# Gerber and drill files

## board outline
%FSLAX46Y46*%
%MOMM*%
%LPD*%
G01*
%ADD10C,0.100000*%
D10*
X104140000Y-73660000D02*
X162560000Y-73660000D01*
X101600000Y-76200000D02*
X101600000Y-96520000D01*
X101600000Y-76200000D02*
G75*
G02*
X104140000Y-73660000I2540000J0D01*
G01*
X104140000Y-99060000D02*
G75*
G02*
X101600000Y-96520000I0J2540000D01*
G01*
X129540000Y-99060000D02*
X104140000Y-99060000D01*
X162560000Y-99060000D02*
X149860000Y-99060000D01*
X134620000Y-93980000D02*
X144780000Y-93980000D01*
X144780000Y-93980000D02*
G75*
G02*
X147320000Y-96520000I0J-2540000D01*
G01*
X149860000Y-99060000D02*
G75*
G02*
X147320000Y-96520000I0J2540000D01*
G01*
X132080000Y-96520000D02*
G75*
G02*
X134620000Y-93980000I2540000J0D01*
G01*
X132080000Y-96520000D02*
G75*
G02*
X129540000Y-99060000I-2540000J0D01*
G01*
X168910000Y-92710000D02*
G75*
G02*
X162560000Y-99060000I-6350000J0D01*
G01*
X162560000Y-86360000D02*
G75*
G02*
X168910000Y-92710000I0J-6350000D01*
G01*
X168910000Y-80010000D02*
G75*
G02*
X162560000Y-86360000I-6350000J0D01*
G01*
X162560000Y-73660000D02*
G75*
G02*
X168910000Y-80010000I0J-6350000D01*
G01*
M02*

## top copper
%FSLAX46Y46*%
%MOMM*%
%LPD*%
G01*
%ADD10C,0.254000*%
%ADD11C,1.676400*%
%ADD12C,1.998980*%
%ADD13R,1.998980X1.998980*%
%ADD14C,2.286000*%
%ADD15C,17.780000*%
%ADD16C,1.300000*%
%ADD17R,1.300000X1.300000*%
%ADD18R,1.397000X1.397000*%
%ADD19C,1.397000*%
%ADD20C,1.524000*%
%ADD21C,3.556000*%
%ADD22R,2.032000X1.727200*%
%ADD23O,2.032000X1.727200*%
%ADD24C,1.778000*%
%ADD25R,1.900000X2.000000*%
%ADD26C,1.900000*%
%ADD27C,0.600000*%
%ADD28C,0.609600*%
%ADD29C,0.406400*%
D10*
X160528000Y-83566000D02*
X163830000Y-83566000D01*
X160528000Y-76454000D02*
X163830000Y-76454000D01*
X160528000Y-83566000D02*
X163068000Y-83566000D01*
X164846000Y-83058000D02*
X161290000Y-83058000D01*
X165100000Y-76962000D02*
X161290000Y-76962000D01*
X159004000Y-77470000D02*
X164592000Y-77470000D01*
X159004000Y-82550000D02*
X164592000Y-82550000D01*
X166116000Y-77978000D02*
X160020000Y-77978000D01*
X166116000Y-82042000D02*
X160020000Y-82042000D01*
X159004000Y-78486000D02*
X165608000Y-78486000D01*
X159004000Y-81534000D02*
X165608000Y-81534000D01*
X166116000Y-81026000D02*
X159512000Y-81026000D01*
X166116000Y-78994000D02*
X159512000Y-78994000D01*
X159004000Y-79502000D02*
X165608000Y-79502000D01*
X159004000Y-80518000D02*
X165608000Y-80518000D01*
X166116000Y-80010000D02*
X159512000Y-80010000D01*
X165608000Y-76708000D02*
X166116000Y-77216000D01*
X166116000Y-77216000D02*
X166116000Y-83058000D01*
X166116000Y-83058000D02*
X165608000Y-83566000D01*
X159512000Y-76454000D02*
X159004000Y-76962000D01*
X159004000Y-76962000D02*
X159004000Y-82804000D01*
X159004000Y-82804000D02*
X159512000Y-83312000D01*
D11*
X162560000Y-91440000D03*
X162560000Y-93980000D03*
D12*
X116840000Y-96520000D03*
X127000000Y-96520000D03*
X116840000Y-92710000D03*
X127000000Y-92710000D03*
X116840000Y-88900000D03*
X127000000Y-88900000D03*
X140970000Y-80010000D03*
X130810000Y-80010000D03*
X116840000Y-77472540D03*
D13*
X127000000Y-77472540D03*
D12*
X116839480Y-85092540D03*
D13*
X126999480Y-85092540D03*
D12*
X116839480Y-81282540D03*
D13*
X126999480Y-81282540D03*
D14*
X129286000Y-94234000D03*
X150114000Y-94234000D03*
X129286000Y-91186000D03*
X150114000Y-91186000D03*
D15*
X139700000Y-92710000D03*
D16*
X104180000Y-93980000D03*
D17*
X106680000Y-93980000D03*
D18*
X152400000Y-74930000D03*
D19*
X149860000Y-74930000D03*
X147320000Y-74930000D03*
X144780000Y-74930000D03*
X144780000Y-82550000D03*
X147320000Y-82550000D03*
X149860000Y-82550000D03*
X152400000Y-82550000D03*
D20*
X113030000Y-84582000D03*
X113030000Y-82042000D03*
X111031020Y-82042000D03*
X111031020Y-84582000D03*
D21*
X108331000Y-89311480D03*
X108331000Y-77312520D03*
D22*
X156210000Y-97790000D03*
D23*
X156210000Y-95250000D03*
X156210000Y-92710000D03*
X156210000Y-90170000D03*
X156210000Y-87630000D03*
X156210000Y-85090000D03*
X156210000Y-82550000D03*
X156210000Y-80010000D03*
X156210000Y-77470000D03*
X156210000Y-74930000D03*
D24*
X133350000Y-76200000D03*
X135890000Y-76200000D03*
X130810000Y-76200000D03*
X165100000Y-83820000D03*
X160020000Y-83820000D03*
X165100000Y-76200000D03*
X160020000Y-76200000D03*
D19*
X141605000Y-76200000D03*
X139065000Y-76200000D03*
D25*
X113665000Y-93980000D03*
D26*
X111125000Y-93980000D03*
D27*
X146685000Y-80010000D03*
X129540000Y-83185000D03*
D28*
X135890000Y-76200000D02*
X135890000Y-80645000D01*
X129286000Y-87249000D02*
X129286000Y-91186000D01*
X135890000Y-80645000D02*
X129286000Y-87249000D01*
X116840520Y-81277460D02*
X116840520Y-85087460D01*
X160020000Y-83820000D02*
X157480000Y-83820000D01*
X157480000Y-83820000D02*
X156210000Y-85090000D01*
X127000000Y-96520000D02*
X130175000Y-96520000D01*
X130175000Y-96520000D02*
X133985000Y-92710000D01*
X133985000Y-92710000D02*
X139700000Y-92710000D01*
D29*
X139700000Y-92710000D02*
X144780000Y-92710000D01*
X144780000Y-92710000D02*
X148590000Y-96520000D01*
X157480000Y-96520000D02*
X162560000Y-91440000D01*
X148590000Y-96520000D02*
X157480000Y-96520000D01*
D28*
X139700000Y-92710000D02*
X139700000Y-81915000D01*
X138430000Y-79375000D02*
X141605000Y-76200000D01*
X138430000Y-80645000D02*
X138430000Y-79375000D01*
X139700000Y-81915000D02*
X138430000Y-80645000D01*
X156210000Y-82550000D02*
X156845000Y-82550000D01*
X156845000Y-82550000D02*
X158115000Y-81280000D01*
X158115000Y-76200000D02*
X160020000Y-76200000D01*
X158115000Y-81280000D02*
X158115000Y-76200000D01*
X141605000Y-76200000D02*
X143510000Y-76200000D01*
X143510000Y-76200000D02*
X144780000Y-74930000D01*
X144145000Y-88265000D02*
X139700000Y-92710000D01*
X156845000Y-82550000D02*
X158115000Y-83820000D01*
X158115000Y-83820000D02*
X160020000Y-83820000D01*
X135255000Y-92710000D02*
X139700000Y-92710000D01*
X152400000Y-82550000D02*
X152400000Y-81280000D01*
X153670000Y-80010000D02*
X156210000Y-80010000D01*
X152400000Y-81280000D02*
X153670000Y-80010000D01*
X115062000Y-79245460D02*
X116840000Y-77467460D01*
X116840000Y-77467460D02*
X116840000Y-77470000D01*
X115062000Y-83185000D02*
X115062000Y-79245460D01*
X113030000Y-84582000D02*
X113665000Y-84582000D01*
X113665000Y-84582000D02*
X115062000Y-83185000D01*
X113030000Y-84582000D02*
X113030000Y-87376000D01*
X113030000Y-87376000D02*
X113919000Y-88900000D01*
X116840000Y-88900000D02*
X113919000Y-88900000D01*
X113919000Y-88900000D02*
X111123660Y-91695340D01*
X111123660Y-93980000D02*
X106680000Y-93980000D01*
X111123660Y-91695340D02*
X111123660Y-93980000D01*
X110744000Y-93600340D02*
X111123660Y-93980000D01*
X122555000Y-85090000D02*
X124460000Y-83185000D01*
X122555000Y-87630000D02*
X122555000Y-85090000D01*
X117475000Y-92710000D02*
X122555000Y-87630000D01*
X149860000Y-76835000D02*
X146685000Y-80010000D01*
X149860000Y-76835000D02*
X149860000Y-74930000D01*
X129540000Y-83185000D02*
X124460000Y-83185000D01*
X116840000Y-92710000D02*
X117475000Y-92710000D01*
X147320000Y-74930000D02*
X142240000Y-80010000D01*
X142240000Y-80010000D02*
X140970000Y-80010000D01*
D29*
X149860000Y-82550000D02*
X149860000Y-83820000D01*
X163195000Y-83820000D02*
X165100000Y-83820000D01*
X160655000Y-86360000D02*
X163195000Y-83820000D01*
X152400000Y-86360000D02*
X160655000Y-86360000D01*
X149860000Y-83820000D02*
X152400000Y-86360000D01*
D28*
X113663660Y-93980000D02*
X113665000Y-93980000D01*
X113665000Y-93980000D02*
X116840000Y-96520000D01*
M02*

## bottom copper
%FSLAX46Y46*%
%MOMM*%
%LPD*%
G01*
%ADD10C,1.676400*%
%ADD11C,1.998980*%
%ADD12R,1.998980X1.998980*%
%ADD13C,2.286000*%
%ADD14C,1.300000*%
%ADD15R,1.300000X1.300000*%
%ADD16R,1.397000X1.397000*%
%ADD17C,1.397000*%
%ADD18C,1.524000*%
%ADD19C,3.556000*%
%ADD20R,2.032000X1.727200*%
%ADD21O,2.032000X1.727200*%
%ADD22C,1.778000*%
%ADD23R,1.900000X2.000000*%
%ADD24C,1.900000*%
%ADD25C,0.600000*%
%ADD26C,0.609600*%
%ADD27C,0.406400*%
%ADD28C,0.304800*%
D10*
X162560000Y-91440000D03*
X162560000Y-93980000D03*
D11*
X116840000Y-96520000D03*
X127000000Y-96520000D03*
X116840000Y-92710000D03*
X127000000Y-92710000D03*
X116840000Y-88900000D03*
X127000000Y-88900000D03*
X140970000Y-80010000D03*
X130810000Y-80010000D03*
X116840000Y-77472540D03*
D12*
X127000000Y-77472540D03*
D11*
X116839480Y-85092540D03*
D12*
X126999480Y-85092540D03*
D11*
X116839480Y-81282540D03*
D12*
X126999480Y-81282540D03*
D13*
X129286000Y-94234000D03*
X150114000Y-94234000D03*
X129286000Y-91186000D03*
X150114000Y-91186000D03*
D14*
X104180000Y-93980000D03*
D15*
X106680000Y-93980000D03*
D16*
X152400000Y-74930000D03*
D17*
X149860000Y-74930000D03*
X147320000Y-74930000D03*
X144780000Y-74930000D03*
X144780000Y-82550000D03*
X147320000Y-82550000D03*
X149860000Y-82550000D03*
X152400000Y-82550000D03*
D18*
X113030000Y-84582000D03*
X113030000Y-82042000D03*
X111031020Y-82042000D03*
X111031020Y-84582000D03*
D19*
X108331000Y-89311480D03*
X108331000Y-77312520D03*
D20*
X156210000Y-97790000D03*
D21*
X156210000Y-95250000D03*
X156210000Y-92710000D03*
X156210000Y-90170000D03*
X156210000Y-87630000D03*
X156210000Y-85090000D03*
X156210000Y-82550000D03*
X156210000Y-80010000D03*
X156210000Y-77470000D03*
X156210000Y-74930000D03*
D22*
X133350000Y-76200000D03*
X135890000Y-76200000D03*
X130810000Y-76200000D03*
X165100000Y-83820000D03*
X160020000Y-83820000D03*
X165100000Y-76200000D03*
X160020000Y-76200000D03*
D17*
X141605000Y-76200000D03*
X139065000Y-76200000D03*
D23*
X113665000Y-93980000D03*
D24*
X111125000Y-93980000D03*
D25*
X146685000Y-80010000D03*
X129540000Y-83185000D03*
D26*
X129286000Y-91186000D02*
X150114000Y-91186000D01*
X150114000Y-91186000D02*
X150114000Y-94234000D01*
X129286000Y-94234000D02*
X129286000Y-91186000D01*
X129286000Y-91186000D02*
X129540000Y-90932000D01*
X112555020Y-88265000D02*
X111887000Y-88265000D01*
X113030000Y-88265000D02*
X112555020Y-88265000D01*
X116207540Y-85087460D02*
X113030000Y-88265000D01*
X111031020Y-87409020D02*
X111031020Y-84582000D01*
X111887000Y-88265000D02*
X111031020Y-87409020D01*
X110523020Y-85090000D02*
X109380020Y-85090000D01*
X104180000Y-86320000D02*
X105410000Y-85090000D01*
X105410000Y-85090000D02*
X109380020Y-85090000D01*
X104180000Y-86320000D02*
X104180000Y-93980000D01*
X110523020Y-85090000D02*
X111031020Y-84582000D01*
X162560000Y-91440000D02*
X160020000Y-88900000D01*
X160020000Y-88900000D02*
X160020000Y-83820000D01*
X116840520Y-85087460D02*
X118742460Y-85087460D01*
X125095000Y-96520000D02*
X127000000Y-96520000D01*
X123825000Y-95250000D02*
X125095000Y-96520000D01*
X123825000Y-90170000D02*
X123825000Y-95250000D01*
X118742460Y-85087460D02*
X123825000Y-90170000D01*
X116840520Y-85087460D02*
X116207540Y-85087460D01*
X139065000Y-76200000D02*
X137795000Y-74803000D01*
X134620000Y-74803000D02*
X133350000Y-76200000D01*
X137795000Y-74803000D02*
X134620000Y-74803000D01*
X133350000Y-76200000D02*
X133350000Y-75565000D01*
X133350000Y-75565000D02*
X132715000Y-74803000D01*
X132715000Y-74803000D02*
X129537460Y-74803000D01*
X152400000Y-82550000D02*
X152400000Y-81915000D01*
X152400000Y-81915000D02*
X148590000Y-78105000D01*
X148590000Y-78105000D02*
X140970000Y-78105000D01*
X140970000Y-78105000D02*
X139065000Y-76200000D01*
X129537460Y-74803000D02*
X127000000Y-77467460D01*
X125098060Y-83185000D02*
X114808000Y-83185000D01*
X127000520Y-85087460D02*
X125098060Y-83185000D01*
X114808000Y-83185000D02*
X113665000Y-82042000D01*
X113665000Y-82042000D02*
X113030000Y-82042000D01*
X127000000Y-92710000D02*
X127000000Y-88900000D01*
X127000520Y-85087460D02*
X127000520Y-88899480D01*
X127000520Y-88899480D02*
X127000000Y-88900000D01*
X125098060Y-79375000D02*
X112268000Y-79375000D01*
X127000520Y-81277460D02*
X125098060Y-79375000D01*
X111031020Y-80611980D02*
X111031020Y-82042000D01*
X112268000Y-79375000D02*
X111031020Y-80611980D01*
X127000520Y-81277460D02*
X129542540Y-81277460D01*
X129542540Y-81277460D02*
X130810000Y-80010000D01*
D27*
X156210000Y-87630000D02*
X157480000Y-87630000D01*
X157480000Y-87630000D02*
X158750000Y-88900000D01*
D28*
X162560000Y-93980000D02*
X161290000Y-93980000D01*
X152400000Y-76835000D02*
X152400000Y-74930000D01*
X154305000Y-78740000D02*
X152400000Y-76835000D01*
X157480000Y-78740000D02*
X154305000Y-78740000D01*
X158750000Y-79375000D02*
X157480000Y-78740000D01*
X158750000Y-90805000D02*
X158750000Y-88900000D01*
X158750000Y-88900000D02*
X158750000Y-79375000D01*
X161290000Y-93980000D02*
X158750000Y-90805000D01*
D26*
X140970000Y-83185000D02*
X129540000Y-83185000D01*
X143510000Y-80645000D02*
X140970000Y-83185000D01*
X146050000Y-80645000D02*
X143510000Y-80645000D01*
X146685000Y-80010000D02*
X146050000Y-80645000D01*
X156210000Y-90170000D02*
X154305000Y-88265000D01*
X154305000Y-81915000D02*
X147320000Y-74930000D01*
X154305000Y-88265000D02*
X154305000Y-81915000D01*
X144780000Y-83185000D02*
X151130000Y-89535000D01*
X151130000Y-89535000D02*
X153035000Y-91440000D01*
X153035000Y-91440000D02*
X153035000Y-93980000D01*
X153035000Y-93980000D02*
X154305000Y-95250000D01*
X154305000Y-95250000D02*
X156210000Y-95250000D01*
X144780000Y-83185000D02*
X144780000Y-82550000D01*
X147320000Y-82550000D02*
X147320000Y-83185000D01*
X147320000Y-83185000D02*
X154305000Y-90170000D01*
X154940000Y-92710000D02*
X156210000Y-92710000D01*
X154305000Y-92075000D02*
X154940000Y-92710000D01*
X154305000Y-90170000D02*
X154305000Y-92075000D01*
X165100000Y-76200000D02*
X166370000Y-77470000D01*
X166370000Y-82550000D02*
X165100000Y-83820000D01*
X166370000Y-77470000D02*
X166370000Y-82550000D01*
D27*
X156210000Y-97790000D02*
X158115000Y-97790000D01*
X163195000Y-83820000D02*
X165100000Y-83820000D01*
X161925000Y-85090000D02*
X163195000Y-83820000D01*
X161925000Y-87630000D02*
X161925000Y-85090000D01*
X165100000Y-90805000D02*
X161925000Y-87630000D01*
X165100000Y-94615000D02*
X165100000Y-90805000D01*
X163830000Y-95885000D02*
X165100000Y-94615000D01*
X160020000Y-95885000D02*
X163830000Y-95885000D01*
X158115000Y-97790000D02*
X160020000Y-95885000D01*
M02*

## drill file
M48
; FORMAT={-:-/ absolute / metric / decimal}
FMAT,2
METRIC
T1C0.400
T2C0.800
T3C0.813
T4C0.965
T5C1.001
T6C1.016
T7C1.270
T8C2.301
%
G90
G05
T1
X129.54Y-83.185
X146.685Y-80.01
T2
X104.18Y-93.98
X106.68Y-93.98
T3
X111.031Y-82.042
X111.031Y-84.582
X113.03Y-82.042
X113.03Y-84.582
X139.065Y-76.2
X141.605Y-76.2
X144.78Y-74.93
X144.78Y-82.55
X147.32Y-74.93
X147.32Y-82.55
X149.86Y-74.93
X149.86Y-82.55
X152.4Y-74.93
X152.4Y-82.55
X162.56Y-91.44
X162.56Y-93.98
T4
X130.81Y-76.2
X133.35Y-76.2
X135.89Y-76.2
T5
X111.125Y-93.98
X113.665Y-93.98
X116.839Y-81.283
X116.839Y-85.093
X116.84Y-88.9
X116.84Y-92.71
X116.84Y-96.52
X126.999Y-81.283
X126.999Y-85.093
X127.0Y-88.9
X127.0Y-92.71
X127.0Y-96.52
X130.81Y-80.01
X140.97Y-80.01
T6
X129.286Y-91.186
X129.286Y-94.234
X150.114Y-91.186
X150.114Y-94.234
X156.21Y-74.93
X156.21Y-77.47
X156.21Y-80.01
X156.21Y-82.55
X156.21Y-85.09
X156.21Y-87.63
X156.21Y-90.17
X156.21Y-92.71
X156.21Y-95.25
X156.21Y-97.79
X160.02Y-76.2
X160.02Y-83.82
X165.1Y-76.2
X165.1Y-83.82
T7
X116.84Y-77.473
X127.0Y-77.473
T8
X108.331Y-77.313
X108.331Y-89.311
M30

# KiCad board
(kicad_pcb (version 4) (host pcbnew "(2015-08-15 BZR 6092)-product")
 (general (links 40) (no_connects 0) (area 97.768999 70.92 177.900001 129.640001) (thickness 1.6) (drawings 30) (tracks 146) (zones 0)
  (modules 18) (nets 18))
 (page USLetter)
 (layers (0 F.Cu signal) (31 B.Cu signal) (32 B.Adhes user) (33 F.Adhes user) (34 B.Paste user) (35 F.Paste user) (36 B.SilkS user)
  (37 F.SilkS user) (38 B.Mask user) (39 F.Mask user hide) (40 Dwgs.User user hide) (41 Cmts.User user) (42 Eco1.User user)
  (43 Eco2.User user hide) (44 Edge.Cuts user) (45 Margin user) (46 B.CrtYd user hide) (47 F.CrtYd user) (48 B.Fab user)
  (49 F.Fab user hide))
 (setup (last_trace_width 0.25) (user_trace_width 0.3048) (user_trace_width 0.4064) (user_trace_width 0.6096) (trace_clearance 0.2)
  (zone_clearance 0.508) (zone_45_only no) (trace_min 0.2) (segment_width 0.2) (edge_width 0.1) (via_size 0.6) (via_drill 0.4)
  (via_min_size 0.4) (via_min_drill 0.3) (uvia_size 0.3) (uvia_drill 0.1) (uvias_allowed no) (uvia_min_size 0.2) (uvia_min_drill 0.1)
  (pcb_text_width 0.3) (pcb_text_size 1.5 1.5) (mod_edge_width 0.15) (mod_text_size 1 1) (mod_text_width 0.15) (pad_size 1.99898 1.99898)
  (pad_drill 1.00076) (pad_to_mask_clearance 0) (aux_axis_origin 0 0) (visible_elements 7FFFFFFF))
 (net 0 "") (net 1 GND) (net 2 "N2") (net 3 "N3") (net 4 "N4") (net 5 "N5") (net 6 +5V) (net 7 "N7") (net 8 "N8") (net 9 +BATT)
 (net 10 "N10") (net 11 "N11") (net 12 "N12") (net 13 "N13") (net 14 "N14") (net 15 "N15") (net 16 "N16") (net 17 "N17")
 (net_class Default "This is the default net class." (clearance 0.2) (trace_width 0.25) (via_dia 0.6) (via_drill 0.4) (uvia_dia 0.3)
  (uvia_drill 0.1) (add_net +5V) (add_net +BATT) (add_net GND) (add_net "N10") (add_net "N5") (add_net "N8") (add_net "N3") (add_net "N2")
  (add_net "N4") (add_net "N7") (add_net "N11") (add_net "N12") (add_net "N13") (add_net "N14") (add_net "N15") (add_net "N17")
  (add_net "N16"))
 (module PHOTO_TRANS (layer F.Cu) (at 162.56 92.71 270)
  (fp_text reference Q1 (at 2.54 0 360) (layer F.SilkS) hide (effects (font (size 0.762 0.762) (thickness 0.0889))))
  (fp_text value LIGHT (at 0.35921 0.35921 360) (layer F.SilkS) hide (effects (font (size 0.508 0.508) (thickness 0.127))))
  (pad 1 thru_hole circle (at -1.27 0 270) (size 1.6764 1.6764) (drill 0.8128) (layers *.Cu *.Mask F.SilkS) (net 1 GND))
  (pad 3 thru_hole circle (at 1.27 0 315) (size 1.6764 1.6764) (drill 0.8128) (layers *.Cu *.Mask F.SilkS) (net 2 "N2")))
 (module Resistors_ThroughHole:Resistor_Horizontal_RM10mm (layer F.Cu) (at 121.92 96.52)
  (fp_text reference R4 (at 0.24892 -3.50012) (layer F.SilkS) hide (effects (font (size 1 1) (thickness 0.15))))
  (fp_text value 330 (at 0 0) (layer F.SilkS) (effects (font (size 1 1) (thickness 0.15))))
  (pad 1 thru_hole circle (at -5.08 0) (size 1.99898 1.99898) (drill 1.00076) (layers *.Cu *.SilkS *.Mask) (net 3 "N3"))
  (pad 2 thru_hole circle (at 5.08 0) (size 1.99898 1.99898) (drill 1.00076) (layers *.Cu *.SilkS *.Mask) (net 1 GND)))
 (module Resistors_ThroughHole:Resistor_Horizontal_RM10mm (layer F.Cu) (at 121.92 92.71)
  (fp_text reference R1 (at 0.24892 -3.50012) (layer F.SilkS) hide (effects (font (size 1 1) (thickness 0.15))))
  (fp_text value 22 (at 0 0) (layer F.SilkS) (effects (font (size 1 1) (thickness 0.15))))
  (pad 1 thru_hole circle (at -5.08 0) (size 1.99898 1.99898) (drill 1.00076) (layers *.Cu *.SilkS *.Mask) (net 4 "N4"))
  (pad 2 thru_hole circle (at 5.08 0) (size 1.99898 1.99898) (drill 1.00076) (layers *.Cu *.SilkS *.Mask) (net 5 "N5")))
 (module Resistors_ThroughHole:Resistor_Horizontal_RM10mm (layer F.Cu) (at 121.92 88.9)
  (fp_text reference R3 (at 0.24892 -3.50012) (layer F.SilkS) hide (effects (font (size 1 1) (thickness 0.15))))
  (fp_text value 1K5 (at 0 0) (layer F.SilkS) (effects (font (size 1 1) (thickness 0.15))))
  (pad 1 thru_hole circle (at -5.08 0) (size 1.99898 1.99898) (drill 1.00076) (layers *.Cu *.SilkS *.Mask) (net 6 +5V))
  (pad 2 thru_hole circle (at 5.08 0) (size 1.99898 1.99898) (drill 1.00076) (layers *.Cu *.SilkS *.Mask) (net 5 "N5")))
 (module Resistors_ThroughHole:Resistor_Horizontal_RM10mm (layer F.Cu) (at 135.89 80.01 180)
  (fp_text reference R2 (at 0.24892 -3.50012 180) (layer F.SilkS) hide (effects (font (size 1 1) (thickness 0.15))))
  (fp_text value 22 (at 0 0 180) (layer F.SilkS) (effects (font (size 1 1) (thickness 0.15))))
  (pad 1 thru_hole circle (at -5.08 0 180) (size 1.99898 1.99898) (drill 1.00076) (layers *.Cu *.SilkS *.Mask) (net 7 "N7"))
  (pad 2 thru_hole circle (at 5.08 0 180) (size 1.99898 1.99898) (drill 1.00076) (layers *.Cu *.SilkS *.Mask) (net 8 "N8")))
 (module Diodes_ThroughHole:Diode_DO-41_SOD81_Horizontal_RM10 (layer F.Cu) (at 127 77.47 180)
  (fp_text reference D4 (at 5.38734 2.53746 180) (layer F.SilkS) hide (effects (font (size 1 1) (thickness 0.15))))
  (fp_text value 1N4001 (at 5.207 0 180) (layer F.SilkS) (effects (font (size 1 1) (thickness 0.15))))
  (pad 2 thru_hole circle (at 10.16 -0.00254) (size 1.99898 1.99898) (drill 1.27) (layers *.Cu *.Mask F.SilkS) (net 6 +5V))
  (pad 1 thru_hole rect (at 0 -0.00254) (size 1.99898 1.99898) (drill 1.27) (layers *.Cu *.Mask F.SilkS) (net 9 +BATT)))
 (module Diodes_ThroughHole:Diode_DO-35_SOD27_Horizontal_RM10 (layer F.Cu) (at 127 85.09 180)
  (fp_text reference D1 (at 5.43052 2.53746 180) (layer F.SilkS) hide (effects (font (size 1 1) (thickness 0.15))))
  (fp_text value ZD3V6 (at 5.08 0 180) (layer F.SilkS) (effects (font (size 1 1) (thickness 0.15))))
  (pad 1 thru_hole circle (at 10.16052 -0.00254) (size 1.99898 1.99898) (drill 1.00076) (layers *.Cu *.Mask F.SilkS) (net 1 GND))
  (pad 2 thru_hole rect (at 0.00052 -0.00254) (size 1.99898 1.99898) (drill 1.00076) (layers *.Cu *.Mask F.SilkS) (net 5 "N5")))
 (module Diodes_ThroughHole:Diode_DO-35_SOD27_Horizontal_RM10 (layer F.Cu) (at 127 81.28 180)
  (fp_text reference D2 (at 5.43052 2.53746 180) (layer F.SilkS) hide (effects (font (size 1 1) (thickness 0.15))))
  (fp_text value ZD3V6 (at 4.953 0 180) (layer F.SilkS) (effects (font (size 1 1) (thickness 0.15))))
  (pad 1 thru_hole circle (at 10.16052 -0.00254) (size 1.99898 1.99898) (drill 1.00076) (layers *.Cu *.Mask F.SilkS) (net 1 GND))
  (pad 2 thru_hole rect (at 0.00052 -0.00254) (size 1.99898 1.99898) (drill 1.00076) (layers *.Cu *.Mask F.SilkS) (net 8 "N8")))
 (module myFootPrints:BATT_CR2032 (layer F.Cu) (at 139.7 92.71)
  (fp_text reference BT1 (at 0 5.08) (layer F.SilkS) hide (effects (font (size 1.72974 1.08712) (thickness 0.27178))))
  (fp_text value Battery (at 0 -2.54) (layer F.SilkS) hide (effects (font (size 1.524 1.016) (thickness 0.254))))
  (pad 1 thru_hole circle (at -10.414 1.524) (size 2.286 2.286) (drill 1.016) (layers *.Cu *.Mask F.SilkS) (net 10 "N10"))
  (pad 1 thru_hole circle (at 10.414 1.524) (size 2.286 2.286) (drill 1.016) (layers *.Cu *.Mask F.SilkS) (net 10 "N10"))
  (pad 1 thru_hole circle (at -10.414 -1.524) (size 2.286 2.286) (drill 1.016) (layers *.Cu *.Mask F.SilkS) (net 10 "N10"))
  (pad 1 thru_hole circle (at 10.414 -1.524) (size 2.286 2.286) (drill 1.016) (layers *.Cu *.Mask F.SilkS) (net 10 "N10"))
  (pad 2 smd circle (at 0 0) (size 17.78 17.78) (layers F.Cu F.Paste F.Mask) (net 1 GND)))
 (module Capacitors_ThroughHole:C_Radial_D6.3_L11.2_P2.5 (layer F.Cu) (at 106.68 93.98 180)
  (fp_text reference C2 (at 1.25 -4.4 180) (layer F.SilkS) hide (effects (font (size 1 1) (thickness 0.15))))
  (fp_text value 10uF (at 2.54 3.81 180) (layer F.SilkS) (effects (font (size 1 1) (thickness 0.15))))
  (pad 2 thru_hole circle (at 2.5 0 180) (size 1.3 1.3) (drill 0.8) (layers *.Cu *.Mask F.SilkS) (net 1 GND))
  (pad 1 thru_hole rect (at 0 0 180) (size 1.3 1.3) (drill 0.8) (layers *.Cu *.Mask F.SilkS) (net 6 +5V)))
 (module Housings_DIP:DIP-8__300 (layer F.Cu) (at 148.59 78.74 180)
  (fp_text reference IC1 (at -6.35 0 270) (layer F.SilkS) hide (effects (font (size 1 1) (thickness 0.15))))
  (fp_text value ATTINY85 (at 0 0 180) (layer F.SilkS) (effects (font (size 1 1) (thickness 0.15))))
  (pad 1 thru_hole rect (at -3.81 3.81 180) (size 1.397 1.397) (drill 0.8128) (layers *.Cu *.Mask F.SilkS) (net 2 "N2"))
  (pad 2 thru_hole circle (at -1.27 3.81 180) (size 1.397 1.397) (drill 0.8128) (layers *.Cu *.Mask F.SilkS) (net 4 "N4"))
  (pad 3 thru_hole circle (at 1.27 3.81 180) (size 1.397 1.397) (drill 0.8128) (layers *.Cu *.Mask F.SilkS) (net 7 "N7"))
  (pad 4 thru_hole circle (at 3.81 3.81 180) (size 1.397 1.397) (drill 0.8128) (layers *.Cu *.Mask F.SilkS) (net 1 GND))
  (pad 5 thru_hole circle (at 3.81 -3.81 180) (size 1.397 1.397) (drill 0.8128) (layers *.Cu *.Mask F.SilkS) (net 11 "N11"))
  (pad 6 thru_hole circle (at 1.27 -3.81 180) (size 1.397 1.397) (drill 0.8128) (layers *.Cu *.Mask F.SilkS) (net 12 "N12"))
  (pad 7 thru_hole circle (at -1.27 -3.81 180) (size 1.397 1.397) (drill 0.8128) (layers *.Cu *.Mask F.SilkS) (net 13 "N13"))
  (pad 8 thru_hole circle (at -3.81 -3.81 180) (size 1.397 1.397) (drill 0.8128) (layers *.Cu *.Mask F.SilkS) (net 9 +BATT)))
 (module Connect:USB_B (layer F.Cu) (at 108.331 83.312 270)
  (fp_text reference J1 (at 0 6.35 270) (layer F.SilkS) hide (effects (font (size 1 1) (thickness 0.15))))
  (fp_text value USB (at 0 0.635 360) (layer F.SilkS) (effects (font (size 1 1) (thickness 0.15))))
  (pad 1 thru_hole circle (at 1.27 -4.699 270) (size 1.524 1.524) (drill 0.8128) (layers *.Cu *.Mask F.SilkS) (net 6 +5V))
  (pad 2 thru_hole circle (at -1.27 -4.699 270) (size 1.524 1.524) (drill 0.8128) (layers *.Cu *.Mask F.SilkS) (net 5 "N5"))
  (pad 3 thru_hole circle (at -1.27 -2.70002 270) (size 1.524 1.524) (drill 0.8128) (layers *.Cu *.Mask F.SilkS) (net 8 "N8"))
  (pad 4 thru_hole circle (at 1.27 -2.70002 270) (size 1.524 1.524) (drill 0.8128) (layers *.Cu *.Mask F.SilkS) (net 1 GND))
  (pad 5 thru_hole circle (at 5.99948 0 270) (size 3.556 3.556) (drill 2.30124) (layers *.Cu *.Mask F.SilkS) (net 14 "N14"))
  (pad 6 thru_hole circle (at -5.99948 0 270) (size 3.556 3.556) (drill 2.30124) (layers *.Cu *.Mask F.SilkS) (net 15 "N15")))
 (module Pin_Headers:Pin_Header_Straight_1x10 (layer F.Cu) (at 156.21 97.79 180)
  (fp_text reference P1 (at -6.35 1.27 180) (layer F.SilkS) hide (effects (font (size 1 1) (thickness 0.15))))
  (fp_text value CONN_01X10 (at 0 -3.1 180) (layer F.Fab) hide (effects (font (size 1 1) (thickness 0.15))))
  (pad 1 thru_hole rect (at 0 0 180) (size 2.032 1.7272) (drill 1.016) (layers *.Cu *.Mask F.SilkS) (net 13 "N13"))
  (pad 2 thru_hole oval (at 0 2.54 180) (size 2.032 1.7272) (drill 1.016) (layers *.Cu *.Mask F.SilkS) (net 11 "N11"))
  (pad 3 thru_hole oval (at 0 5.08 180) (size 2.032 1.7272) (drill 1.016) (layers *.Cu *.Mask F.SilkS) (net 12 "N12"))
  (pad 4 thru_hole oval (at 0 7.62 180) (size 2.032 1.7272) (drill 1.016) (layers *.Cu *.Mask F.SilkS) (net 7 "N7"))
  (pad 5 thru_hole oval (at 0 10.16 180) (size 2.032 1.7272) (drill 1.016) (layers *.Cu *.Mask F.SilkS) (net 2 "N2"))
  (pad 6 thru_hole oval (at 0 12.7 180) (size 2.032 1.7272) (drill 1.016) (layers *.Cu *.Mask F.SilkS) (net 1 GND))
  (pad 7 thru_hole oval (at 0 15.24 180) (size 2.032 1.7272) (drill 1.016) (layers *.Cu *.Mask F.SilkS) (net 1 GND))
  (pad 8 thru_hole oval (at 0 17.78 180) (size 2.032 1.7272) (drill 1.016) (layers *.Cu *.Mask F.SilkS) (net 9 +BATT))
  (pad 9 thru_hole oval (at 0 20.32 180) (size 2.032 1.7272) (drill 1.016) (layers *.Cu *.Mask F.SilkS) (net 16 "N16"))
  (pad 10 thru_hole oval (at 0 22.86 180) (size 2.032 1.7272) (drill 1.016) (layers *.Cu *.Mask F.SilkS) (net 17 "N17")))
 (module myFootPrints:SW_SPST (layer F.Cu) (at 133.35 76.2 270)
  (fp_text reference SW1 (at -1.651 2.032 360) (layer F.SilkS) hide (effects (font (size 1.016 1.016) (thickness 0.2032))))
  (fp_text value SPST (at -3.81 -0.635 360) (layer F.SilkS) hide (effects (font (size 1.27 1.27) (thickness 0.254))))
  (pad 2 thru_hole circle (at 0 0 270) (size 1.778 1.778) (drill 0.9652) (layers *.Cu *.Mask F.SilkS) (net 9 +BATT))
  (pad 1 thru_hole circle (at 0 -2.54 270) (size 1.778 1.778) (drill 0.9652) (layers *.Cu *.Mask F.SilkS) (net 10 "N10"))
  (pad 3 thru_hole circle (at 0 2.54 270) (size 1.778 1.778) (drill 0.9652) (layers *.Cu *.Mask F.SilkS)))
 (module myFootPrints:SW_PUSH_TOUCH (layer F.Cu) (at 162.56 80.01 270)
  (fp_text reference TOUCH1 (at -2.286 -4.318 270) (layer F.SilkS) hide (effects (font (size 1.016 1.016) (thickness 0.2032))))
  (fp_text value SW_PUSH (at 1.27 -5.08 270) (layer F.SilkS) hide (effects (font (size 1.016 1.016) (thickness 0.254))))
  (fp_line (start 3.556 2.032) (end 3.556 -1.27) (layer F.Cu) (width 0.254))
  (fp_line (start -3.556 2.032) (end -3.556 -1.27) (layer F.Cu) (width 0.254))
  (fp_line (start 3.556 2.032) (end 3.556 -0.508) (layer F.Cu) (width 0.254))
  (fp_line (start 3.048 -2.286) (end 3.048 1.27) (layer F.Cu) (width 0.254))
  (fp_line (start -3.048 -2.54) (end -3.048 1.27) (layer F.Cu) (width 0.254))
  (fp_line (start -2.54 3.556) (end -2.54 -2.032) (layer F.Cu) (width 0.254))
  (fp_line (start 2.54 3.556) (end 2.54 -2.032) (layer F.Cu) (width 0.254))
  (fp_line (start -2.032 -3.556) (end -2.032 2.54) (layer F.Cu) (width 0.254))
  (fp_line (start 2.032 -3.556) (end 2.032 2.54) (layer F.Cu) (width 0.254))
  (fp_line (start -1.524 3.556) (end -1.524 -3.048) (layer F.Cu) (width 0.254))
  (fp_line (start 1.524 3.556) (end 1.524 -3.048) (layer F.Cu) (width 0.254))
  (fp_line (start 1.016 -3.556) (end 1.016 3.048) (layer F.Cu) (width 0.254))
  (fp_line (start -1.016 -3.556) (end -1.016 3.048) (layer F.Cu) (width 0.254))
  (fp_line (start -0.508 3.556) (end -0.508 -3.048) (layer F.Cu) (width 0.254))
  (fp_line (start 0.508 3.556) (end 0.508 -3.048) (layer F.Cu) (width 0.254))
  (fp_line (start 0 -3.556) (end 0 3.048) (layer F.Cu) (width 0.254))
  (fp_line (start -3.302 -3.048) (end -2.794 -3.556) (layer F.Cu) (width 0.254))
  (fp_line (start -2.794 -3.556) (end 3.048 -3.556) (layer F.Cu) (width 0.254))
  (fp_line (start 3.048 -3.556) (end 3.556 -3.048) (layer F.Cu) (width 0.254))
  (fp_line (start -3.556 3.048) (end -3.048 3.556) (layer F.Cu) (width 0.254))
  (fp_line (start -3.048 3.556) (end 2.794 3.556) (layer F.Cu) (width 0.254))
  (fp_line (start 2.794 3.556) (end 3.302 3.048) (layer F.Cu) (width 0.254))
  (pad 1 thru_hole circle (at 3.81 -2.54 270) (size 1.778 1.778) (drill 1.016) (layers *.Cu *.Mask F.SilkS) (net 13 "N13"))
  (pad 2 thru_hole circle (at 3.81 2.54 270) (size 1.778 1.778) (drill 1.016) (layers *.Cu *.Mask F.SilkS) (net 1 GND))
  (pad 1 thru_hole circle (at -3.81 -2.54 270) (size 1.778 1.778) (drill 1.016) (layers *.Cu *.Mask F.SilkS) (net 13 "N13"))
  (pad 2 thru_hole circle (at -3.81 2.54 270) (size 1.778 1.778) (drill 1.016) (layers *.Cu *.Mask F.SilkS) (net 1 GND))
  (pad 3 smd circle (at 0 0 270) (size 7.62 7.62) (layers F.Paste F.Mask)))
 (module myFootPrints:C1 (layer F.Cu) (at 140.335 76.2 180)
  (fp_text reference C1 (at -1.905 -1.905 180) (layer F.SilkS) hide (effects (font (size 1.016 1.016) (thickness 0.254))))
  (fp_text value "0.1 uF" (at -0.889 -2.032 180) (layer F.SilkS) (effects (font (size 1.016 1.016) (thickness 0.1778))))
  (pad 1 thru_hole circle (at -1.27 0 180) (size 1.397 1.397) (drill 0.8128) (layers *.Cu *.Mask F.SilkS) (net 1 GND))
  (pad 2 thru_hole circle (at 1.27 0 180) (size 1.397 1.397) (drill 0.8128) (layers *.Cu *.Mask F.SilkS) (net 9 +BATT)))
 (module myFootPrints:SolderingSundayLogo (layer F.Cu) (at 141.605 85.979)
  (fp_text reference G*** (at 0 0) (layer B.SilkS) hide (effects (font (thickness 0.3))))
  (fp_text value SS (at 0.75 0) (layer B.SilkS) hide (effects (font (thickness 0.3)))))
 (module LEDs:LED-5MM (layer F.Cu) (at 113.665 93.98 180)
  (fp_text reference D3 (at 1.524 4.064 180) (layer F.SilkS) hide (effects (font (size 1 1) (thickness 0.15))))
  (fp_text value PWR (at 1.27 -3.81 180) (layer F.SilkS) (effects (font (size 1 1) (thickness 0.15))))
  (pad 1 thru_hole rect (at 0 0 270) (size 2 1.9) (drill 1.00076) (layers *.Cu *.Mask F.SilkS) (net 3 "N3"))
  (pad 2 thru_hole circle (at 2.54 0 180) (size 1.9 1.9) (drill 1.00076) (layers *.Cu *.Mask F.SilkS) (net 6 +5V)))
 (gr_line (start 104.14 73.66) (end 162.56 73.66) (angle 90) (layer Edge.Cuts) (width 0.1))
 (gr_line (start 101.6 76.2) (end 101.6 96.52) (angle 90) (layer Edge.Cuts) (width 0.1))
 (gr_arc (start 104.14 76.2) (end 101.6 76.2) (angle 90) (layer Edge.Cuts) (width 0.1))
 (gr_arc (start 104.14 96.52) (end 104.14 99.06) (angle 90) (layer Edge.Cuts) (width 0.1))
 (gr_line (start 129.54 99.06) (end 104.14 99.06) (angle 90) (layer Edge.Cuts) (width 0.1))
 (gr_line (start 162.56 99.06) (end 149.86 99.06) (angle 90) (layer Edge.Cuts) (width 0.1))
 (gr_line (start 134.62 93.98) (end 144.78 93.98) (angle 90) (layer Edge.Cuts) (width 0.1))
 (gr_arc (start 144.78 96.52) (end 144.78 93.98) (angle 90) (layer Edge.Cuts) (width 0.1))
 (gr_arc (start 149.86 96.52) (end 149.86 99.06) (angle 90) (layer Edge.Cuts) (width 0.1))
 (gr_arc (start 134.62 96.52) (end 132.08 96.52) (angle 90) (layer Edge.Cuts) (width 0.1))
 (gr_arc (start 129.54 96.52) (end 132.08 96.52) (angle 90) (layer Edge.Cuts) (width 0.1))
 (gr_arc (start 162.56 92.71) (end 168.91 92.71) (angle 90) (layer Edge.Cuts) (width 0.1))
 (gr_arc (start 162.56 92.71) (end 162.56 86.36) (angle 90) (layer Edge.Cuts) (width 0.1))
 (gr_arc (start 162.56 80.01) (end 168.91 80.01) (angle 90) (layer Edge.Cuts) (width 0.1))
 (gr_arc (start 162.56 80.01) (end 162.56 73.66) (angle 90) (layer Edge.Cuts) (width 0.1))
 (segment (start 135.89 76.2) (end 135.89 80.645) (width 0.6096) (layer F.Cu) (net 10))
 (segment (start 129.286 87.249) (end 129.286 91.186) (width 0.6096) (layer F.Cu) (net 10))
 (segment (start 135.89 80.645) (end 129.286 87.249) (width 0.6096) (layer F.Cu) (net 10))
 (segment (start 129.286 91.186) (end 150.114 91.186) (width 0.6096) (layer B.Cu) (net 10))
 (segment (start 150.114 91.186) (end 150.114 94.234) (width 0.6096) (layer B.Cu) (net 10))
 (segment (start 129.286 94.234) (end 129.286 91.186) (width 0.6096) (layer B.Cu) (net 10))
 (segment (start 129.286 91.186) (end 129.54 90.932) (width 0.6096) (layer B.Cu) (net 10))
 (segment (start 116.84052 81.27746) (end 116.84052 85.08746) (width 0.6096) (layer F.Cu) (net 1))
 (segment (start 160.02 83.82) (end 157.48 83.82) (width 0.6096) (layer F.Cu) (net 1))
 (segment (start 157.48 83.82) (end 156.21 85.09) (width 0.6096) (layer F.Cu) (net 1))
 (segment (start 127 96.52) (end 130.175 96.52) (width 0.6096) (layer F.Cu) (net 1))
 (segment (start 130.175 96.52) (end 133.985 92.71) (width 0.6096) (layer F.Cu) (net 1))
 (segment (start 133.985 92.71) (end 139.7 92.71) (width 0.6096) (layer F.Cu) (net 1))
 (segment (start 112.55502 88.265) (end 111.887 88.265) (width 0.6096) (layer B.Cu) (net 1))
 (segment (start 113.03 88.265) (end 112.55502 88.265) (width 0.6096) (layer B.Cu) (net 1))
 (segment (start 116.20754 85.08746) (end 113.03 88.265) (width 0.6096) (layer B.Cu) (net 1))
 (segment (start 111.03102 87.40902) (end 111.03102 84.582) (width 0.6096) (layer B.Cu) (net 1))
 (segment (start 111.887 88.265) (end 111.03102 87.40902) (width 0.6096) (layer B.Cu) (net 1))
 (segment (start 110.52302 85.09) (end 109.38002 85.09) (width 0.6096) (layer B.Cu) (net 1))
 (segment (start 104.18 86.32) (end 105.41 85.09) (width 0.6096) (layer B.Cu) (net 1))
 (segment (start 105.41 85.09) (end 109.38002 85.09) (width 0.6096) (layer B.Cu) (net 1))
 (segment (start 104.18 86.32) (end 104.18 93.98) (width 0.6096) (layer B.Cu) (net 1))
 (segment (start 110.52302 85.09) (end 111.03102 84.582) (width 0.6096) (layer B.Cu) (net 1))
 (segment (start 162.56 91.44) (end 160.02 88.9) (width 0.6096) (layer B.Cu) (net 1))
 (segment (start 160.02 88.9) (end 160.02 83.82) (width 0.6096) (layer B.Cu) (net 1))
 (segment (start 139.7 92.71) (end 144.78 92.71) (width 0.4064) (layer F.Cu) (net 1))
 (segment (start 144.78 92.71) (end 148.59 96.52) (width 0.4064) (layer F.Cu) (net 1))
 (segment (start 157.48 96.52) (end 162.56 91.44) (width 0.4064) (layer F.Cu) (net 1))
 (segment (start 148.59 96.52) (end 157.48 96.52) (width 0.4064) (layer F.Cu) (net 1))
 (segment (start 139.7 92.71) (end 139.7 81.915) (width 0.6096) (layer F.Cu) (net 1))
 (segment (start 138.43 79.375) (end 141.605 76.2) (width 0.6096) (layer F.Cu) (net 1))
 (segment (start 138.43 80.645) (end 138.43 79.375) (width 0.6096) (layer F.Cu) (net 1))
 (segment (start 139.7 81.915) (end 138.43 80.645) (width 0.6096) (layer F.Cu) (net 1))
 (segment (start 156.21 82.55) (end 156.845 82.55) (width 0.6096) (layer F.Cu) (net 1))
 (segment (start 156.845 82.55) (end 158.115 81.28) (width 0.6096) (layer F.Cu) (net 1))
 (segment (start 158.115 76.2) (end 160.02 76.2) (width 0.6096) (layer F.Cu) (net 1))
 (segment (start 158.115 81.28) (end 158.115 76.2) (width 0.6096) (layer F.Cu) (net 1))
 (segment (start 141.605 76.2) (end 143.51 76.2) (width 0.6096) (layer F.Cu) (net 1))
 (segment (start 143.51 76.2) (end 144.78 74.93) (width 0.6096) (layer F.Cu) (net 1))
 (segment (start 144.145 88.265) (end 139.7 92.71) (width 0.6096) (layer F.Cu) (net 1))
 (segment (start 156.845 82.55) (end 158.115 83.82) (width 0.6096) (layer F.Cu) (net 1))
 (segment (start 158.115 83.82) (end 160.02 83.82) (width 0.6096) (layer F.Cu) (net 1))
 (segment (start 135.255 92.71) (end 139.7 92.71) (width 0.6096) (layer F.Cu) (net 1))
 (segment (start 116.84052 85.08746) (end 118.74246 85.08746) (width 0.6096) (layer B.Cu) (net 1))
 (segment (start 125.095 96.52) (end 127 96.52) (width 0.6096) (layer B.Cu) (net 1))
 (segment (start 123.825 95.25) (end 125.095 96.52) (width 0.6096) (layer B.Cu) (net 1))
 (segment (start 123.825 90.17) (end 123.825 95.25) (width 0.6096) (layer B.Cu) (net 1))
 (segment (start 118.74246 85.08746) (end 123.825 90.17) (width 0.6096) (layer B.Cu) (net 1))
 (segment (start 116.84052 85.08746) (end 116.20754 85.08746) (width 0.6096) (layer B.Cu) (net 1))
 (segment (start 152.4 82.55) (end 152.4 81.28) (width 0.6096) (layer F.Cu) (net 9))
 (segment (start 153.67 80.01) (end 156.21 80.01) (width 0.6096) (layer F.Cu) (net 9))
 (segment (start 152.4 81.28) (end 153.67 80.01) (width 0.6096) (layer F.Cu) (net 9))
 (segment (start 139.065 76.2) (end 137.795 74.803) (width 0.6096) (layer B.Cu) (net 9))
 (segment (start 134.62 74.803) (end 133.35 76.2) (width 0.6096) (layer B.Cu) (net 9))
 (segment (start 137.795 74.803) (end 134.62 74.803) (width 0.6096) (layer B.Cu) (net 9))
 (segment (start 133.35 76.2) (end 133.35 75.565) (width 0.6096) (layer B.Cu) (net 9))
 (segment (start 133.35 75.565) (end 132.715 74.803) (width 0.6096) (layer B.Cu) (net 9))
 (segment (start 132.715 74.803) (end 129.53746 74.803) (width 0.6096) (layer B.Cu) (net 9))
 (segment (start 152.4 82.55) (end 152.4 81.915) (width 0.6096) (layer B.Cu) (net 9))
 (segment (start 152.4 81.915) (end 148.59 78.105) (width 0.6096) (layer B.Cu) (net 9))
 (segment (start 148.59 78.105) (end 140.97 78.105) (width 0.6096) (layer B.Cu) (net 9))
 (segment (start 140.97 78.105) (end 139.065 76.2) (width 0.6096) (layer B.Cu) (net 9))
 (segment (start 129.53746 74.803) (end 127 77.46746) (width 0.6096) (layer B.Cu) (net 9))
 (segment (start 115.062 79.24546) (end 116.84 77.46746) (width 0.6096) (layer F.Cu) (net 6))
 (segment (start 116.84 77.46746) (end 116.84 77.47) (width 0.6096) (layer F.Cu) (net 6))
 (segment (start 115.062 83.185) (end 115.062 79.24546) (width 0.6096) (layer F.Cu) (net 6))
 (segment (start 113.03 84.582) (end 113.665 84.582) (width 0.6096) (layer F.Cu) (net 6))
 (segment (start 113.665 84.582) (end 115.062 83.185) (width 0.6096) (layer F.Cu) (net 6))
 (segment (start 113.03 84.582) (end 113.03 87.376) (width 0.6096) (layer F.Cu) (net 6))
 (segment (start 113.03 87.376) (end 113.919 88.9) (width 0.6096) (layer F.Cu) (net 6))
 (segment (start 116.84 88.9) (end 113.919 88.9) (width 0.6096) (layer F.Cu) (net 6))
 (segment (start 113.919 88.9) (end 111.12366 91.69534) (width 0.6096) (layer F.Cu) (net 6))
 (segment (start 111.12366 93.98) (end 106.68 93.98) (width 0.6096) (layer F.Cu) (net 6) (status 10))
 (segment (start 111.12366 91.69534) (end 111.12366 93.98) (width 0.6096) (layer F.Cu) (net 6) (status 20))
 (segment (start 110.744 93.60034) (end 111.12366 93.98) (width 0.6096) (layer F.Cu) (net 6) (status 30))
 (segment (start 125.09806 83.185) (end 114.808 83.185) (width 0.6096) (layer B.Cu) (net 5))
 (segment (start 127.00052 85.08746) (end 125.09806 83.185) (width 0.6096) (layer B.Cu) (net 5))
 (segment (start 114.808 83.185) (end 113.665 82.042) (width 0.6096) (layer B.Cu) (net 5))
 (segment (start 113.665 82.042) (end 113.03 82.042) (width 0.6096) (layer B.Cu) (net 5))
 (segment (start 127 92.71) (end 127 88.9) (width 0.6096) (layer B.Cu) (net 5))
 (segment (start 127.00052 85.08746) (end 127.00052 88.89948) (width 0.6096) (layer B.Cu) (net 5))
 (segment (start 127.00052 88.89948) (end 127 88.9) (width 0.6096) (layer B.Cu) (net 5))
 (segment (start 125.09806 79.375) (end 112.268 79.375) (width 0.6096) (layer B.Cu) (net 8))
 (segment (start 127.00052 81.27746) (end 125.09806 79.375) (width 0.6096) (layer B.Cu) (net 8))
 (segment (start 111.03102 80.61198) (end 111.03102 82.042) (width 0.6096) (layer B.Cu) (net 8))
 (segment (start 112.268 79.375) (end 111.03102 80.61198) (width 0.6096) (layer B.Cu) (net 8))
 (segment (start 127.00052 81.27746) (end 129.54254 81.27746) (width 0.6096) (layer B.Cu) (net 8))
 (segment (start 129.54254 81.27746) (end 130.81 80.01) (width 0.6096) (layer B.Cu) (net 8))
 (segment (start 156.21 87.63) (end 157.48 87.63) (width 0.4064) (layer B.Cu) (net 2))
 (segment (start 157.48 87.63) (end 158.75 88.9) (width 0.4064) (layer B.Cu) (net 2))
 (segment (start 162.56 93.98) (end 161.29 93.98) (width 0.3048) (layer B.Cu) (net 2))
 (segment (start 152.4 76.835) (end 152.4 74.93) (width 0.3048) (layer B.Cu) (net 2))
 (segment (start 154.305 78.74) (end 152.4 76.835) (width 0.3048) (layer B.Cu) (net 2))
 (segment (start 157.48 78.74) (end 154.305 78.74) (width 0.3048) (layer B.Cu) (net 2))
 (segment (start 158.75 79.375) (end 157.48 78.74) (width 0.3048) (layer B.Cu) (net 2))
 (segment (start 158.75 90.805) (end 158.75 88.9) (width 0.3048) (layer B.Cu) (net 2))
 (segment (start 158.75 88.9) (end 158.75 79.375) (width 0.3048) (layer B.Cu) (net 2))
 (segment (start 161.29 93.98) (end 158.75 90.805) (width 0.3048) (layer B.Cu) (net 2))
 (via (at 146.685 80.01) (size 0.6) (layers F.Cu B.Cu) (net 4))
 (segment (start 122.555 85.09) (end 124.46 83.185) (width 0.6096) (layer F.Cu) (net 4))
 (segment (start 122.555 87.63) (end 122.555 85.09) (width 0.6096) (layer F.Cu) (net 4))
 (segment (start 117.475 92.71) (end 122.555 87.63) (width 0.6096) (layer F.Cu) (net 4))
 (segment (start 149.86 76.835) (end 146.685 80.01) (width 0.6096) (layer F.Cu) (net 4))
 (segment (start 149.86 76.835) (end 149.86 74.93) (width 0.6096) (layer F.Cu) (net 4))
 (segment (start 129.54 83.185) (end 124.46 83.185) (width 0.6096) (layer F.Cu) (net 4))
 (via (at 129.54 83.185) (size 0.6) (layers F.Cu B.Cu) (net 4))
 (segment (start 140.97 83.185) (end 129.54 83.185) (width 0.6096) (layer B.Cu) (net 4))
 (segment (start 143.51 80.645) (end 140.97 83.185) (width 0.6096) (layer B.Cu) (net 4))
 (segment (start 146.05 80.645) (end 143.51 80.645) (width 0.6096) (layer B.Cu) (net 4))
 (segment (start 146.685 80.01) (end 146.05 80.645) (width 0.6096) (layer B.Cu) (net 4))
 (segment (start 116.84 92.71) (end 117.475 92.71) (width 0.6096) (layer F.Cu) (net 4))
 (segment (start 147.32 74.93) (end 142.24 80.01) (width 0.6096) (layer F.Cu) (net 7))
 (segment (start 142.24 80.01) (end 140.97 80.01) (width 0.6096) (layer F.Cu) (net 7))
 (segment (start 156.21 90.17) (end 154.305 88.265) (width 0.6096) (layer B.Cu) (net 7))
 (segment (start 154.305 81.915) (end 147.32 74.93) (width 0.6096) (layer B.Cu) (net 7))
 (segment (start 154.305 88.265) (end 154.305 81.915) (width 0.6096) (layer B.Cu) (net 7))
 (segment (start 144.78 83.185) (end 151.13 89.535) (width 0.6096) (layer B.Cu) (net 11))
 (segment (start 151.13 89.535) (end 153.035 91.44) (width 0.6096) (layer B.Cu) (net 11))
 (segment (start 153.035 91.44) (end 153.035 93.98) (width 0.6096) (layer B.Cu) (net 11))
 (segment (start 153.035 93.98) (end 154.305 95.25) (width 0.6096) (layer B.Cu) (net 11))
 (segment (start 154.305 95.25) (end 156.21 95.25) (width 0.6096) (layer B.Cu) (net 11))
 (segment (start 144.78 83.185) (end 144.78 82.55) (width 0.6096) (layer B.Cu) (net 11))
 (segment (start 147.32 82.55) (end 147.32 83.185) (width 0.6096) (layer B.Cu) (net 12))
 (segment (start 147.32 83.185) (end 154.305 90.17) (width 0.6096) (layer B.Cu) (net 12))
 (segment (start 154.94 92.71) (end 156.21 92.71) (width 0.6096) (layer B.Cu) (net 12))
 (segment (start 154.305 92.075) (end 154.94 92.71) (width 0.6096) (layer B.Cu) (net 12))
 (segment (start 154.305 90.17) (end 154.305 92.075) (width 0.6096) (layer B.Cu) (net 12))
 (segment (start 165.1 76.2) (end 166.37 77.47) (width 0.6096) (layer B.Cu) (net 13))
 (segment (start 166.37 82.55) (end 165.1 83.82) (width 0.6096) (layer B.Cu) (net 13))
 (segment (start 166.37 77.47) (end 166.37 82.55) (width 0.6096) (layer B.Cu) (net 13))
 (segment (start 149.86 82.55) (end 149.86 83.82) (width 0.4064) (layer F.Cu) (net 13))
 (segment (start 163.195 83.82) (end 165.1 83.82) (width 0.4064) (layer F.Cu) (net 13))
 (segment (start 160.655 86.36) (end 163.195 83.82) (width 0.4064) (layer F.Cu) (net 13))
 (segment (start 152.4 86.36) (end 160.655 86.36) (width 0.4064) (layer F.Cu) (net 13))
 (segment (start 149.86 83.82) (end 152.4 86.36) (width 0.4064) (layer F.Cu) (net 13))
 (segment (start 156.21 97.79) (end 158.115 97.79) (width 0.4064) (layer B.Cu) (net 13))
 (segment (start 163.195 83.82) (end 165.1 83.82) (width 0.4064) (layer B.Cu) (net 13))
 (segment (start 161.925 85.09) (end 163.195 83.82) (width 0.4064) (layer B.Cu) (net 13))
 (segment (start 161.925 87.63) (end 161.925 85.09) (width 0.4064) (layer B.Cu) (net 13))
 (segment (start 165.1 90.805) (end 161.925 87.63) (width 0.4064) (layer B.Cu) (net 13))
 (segment (start 165.1 94.615) (end 165.1 90.805) (width 0.4064) (layer B.Cu) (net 13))
 (segment (start 163.83 95.885) (end 165.1 94.615) (width 0.4064) (layer B.Cu) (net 13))
 (segment (start 160.02 95.885) (end 163.83 95.885) (width 0.4064) (layer B.Cu) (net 13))
 (segment (start 158.115 97.79) (end 160.02 95.885) (width 0.4064) (layer B.Cu) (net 13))
 (segment (start 113.66366 93.98) (end 113.665 93.98) (width 0.6096) (layer F.Cu) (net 3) (status 30))
 (segment (start 113.665 93.98) (end 116.84 96.52) (width 0.6096) (layer F.Cu) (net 3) (status 10)))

